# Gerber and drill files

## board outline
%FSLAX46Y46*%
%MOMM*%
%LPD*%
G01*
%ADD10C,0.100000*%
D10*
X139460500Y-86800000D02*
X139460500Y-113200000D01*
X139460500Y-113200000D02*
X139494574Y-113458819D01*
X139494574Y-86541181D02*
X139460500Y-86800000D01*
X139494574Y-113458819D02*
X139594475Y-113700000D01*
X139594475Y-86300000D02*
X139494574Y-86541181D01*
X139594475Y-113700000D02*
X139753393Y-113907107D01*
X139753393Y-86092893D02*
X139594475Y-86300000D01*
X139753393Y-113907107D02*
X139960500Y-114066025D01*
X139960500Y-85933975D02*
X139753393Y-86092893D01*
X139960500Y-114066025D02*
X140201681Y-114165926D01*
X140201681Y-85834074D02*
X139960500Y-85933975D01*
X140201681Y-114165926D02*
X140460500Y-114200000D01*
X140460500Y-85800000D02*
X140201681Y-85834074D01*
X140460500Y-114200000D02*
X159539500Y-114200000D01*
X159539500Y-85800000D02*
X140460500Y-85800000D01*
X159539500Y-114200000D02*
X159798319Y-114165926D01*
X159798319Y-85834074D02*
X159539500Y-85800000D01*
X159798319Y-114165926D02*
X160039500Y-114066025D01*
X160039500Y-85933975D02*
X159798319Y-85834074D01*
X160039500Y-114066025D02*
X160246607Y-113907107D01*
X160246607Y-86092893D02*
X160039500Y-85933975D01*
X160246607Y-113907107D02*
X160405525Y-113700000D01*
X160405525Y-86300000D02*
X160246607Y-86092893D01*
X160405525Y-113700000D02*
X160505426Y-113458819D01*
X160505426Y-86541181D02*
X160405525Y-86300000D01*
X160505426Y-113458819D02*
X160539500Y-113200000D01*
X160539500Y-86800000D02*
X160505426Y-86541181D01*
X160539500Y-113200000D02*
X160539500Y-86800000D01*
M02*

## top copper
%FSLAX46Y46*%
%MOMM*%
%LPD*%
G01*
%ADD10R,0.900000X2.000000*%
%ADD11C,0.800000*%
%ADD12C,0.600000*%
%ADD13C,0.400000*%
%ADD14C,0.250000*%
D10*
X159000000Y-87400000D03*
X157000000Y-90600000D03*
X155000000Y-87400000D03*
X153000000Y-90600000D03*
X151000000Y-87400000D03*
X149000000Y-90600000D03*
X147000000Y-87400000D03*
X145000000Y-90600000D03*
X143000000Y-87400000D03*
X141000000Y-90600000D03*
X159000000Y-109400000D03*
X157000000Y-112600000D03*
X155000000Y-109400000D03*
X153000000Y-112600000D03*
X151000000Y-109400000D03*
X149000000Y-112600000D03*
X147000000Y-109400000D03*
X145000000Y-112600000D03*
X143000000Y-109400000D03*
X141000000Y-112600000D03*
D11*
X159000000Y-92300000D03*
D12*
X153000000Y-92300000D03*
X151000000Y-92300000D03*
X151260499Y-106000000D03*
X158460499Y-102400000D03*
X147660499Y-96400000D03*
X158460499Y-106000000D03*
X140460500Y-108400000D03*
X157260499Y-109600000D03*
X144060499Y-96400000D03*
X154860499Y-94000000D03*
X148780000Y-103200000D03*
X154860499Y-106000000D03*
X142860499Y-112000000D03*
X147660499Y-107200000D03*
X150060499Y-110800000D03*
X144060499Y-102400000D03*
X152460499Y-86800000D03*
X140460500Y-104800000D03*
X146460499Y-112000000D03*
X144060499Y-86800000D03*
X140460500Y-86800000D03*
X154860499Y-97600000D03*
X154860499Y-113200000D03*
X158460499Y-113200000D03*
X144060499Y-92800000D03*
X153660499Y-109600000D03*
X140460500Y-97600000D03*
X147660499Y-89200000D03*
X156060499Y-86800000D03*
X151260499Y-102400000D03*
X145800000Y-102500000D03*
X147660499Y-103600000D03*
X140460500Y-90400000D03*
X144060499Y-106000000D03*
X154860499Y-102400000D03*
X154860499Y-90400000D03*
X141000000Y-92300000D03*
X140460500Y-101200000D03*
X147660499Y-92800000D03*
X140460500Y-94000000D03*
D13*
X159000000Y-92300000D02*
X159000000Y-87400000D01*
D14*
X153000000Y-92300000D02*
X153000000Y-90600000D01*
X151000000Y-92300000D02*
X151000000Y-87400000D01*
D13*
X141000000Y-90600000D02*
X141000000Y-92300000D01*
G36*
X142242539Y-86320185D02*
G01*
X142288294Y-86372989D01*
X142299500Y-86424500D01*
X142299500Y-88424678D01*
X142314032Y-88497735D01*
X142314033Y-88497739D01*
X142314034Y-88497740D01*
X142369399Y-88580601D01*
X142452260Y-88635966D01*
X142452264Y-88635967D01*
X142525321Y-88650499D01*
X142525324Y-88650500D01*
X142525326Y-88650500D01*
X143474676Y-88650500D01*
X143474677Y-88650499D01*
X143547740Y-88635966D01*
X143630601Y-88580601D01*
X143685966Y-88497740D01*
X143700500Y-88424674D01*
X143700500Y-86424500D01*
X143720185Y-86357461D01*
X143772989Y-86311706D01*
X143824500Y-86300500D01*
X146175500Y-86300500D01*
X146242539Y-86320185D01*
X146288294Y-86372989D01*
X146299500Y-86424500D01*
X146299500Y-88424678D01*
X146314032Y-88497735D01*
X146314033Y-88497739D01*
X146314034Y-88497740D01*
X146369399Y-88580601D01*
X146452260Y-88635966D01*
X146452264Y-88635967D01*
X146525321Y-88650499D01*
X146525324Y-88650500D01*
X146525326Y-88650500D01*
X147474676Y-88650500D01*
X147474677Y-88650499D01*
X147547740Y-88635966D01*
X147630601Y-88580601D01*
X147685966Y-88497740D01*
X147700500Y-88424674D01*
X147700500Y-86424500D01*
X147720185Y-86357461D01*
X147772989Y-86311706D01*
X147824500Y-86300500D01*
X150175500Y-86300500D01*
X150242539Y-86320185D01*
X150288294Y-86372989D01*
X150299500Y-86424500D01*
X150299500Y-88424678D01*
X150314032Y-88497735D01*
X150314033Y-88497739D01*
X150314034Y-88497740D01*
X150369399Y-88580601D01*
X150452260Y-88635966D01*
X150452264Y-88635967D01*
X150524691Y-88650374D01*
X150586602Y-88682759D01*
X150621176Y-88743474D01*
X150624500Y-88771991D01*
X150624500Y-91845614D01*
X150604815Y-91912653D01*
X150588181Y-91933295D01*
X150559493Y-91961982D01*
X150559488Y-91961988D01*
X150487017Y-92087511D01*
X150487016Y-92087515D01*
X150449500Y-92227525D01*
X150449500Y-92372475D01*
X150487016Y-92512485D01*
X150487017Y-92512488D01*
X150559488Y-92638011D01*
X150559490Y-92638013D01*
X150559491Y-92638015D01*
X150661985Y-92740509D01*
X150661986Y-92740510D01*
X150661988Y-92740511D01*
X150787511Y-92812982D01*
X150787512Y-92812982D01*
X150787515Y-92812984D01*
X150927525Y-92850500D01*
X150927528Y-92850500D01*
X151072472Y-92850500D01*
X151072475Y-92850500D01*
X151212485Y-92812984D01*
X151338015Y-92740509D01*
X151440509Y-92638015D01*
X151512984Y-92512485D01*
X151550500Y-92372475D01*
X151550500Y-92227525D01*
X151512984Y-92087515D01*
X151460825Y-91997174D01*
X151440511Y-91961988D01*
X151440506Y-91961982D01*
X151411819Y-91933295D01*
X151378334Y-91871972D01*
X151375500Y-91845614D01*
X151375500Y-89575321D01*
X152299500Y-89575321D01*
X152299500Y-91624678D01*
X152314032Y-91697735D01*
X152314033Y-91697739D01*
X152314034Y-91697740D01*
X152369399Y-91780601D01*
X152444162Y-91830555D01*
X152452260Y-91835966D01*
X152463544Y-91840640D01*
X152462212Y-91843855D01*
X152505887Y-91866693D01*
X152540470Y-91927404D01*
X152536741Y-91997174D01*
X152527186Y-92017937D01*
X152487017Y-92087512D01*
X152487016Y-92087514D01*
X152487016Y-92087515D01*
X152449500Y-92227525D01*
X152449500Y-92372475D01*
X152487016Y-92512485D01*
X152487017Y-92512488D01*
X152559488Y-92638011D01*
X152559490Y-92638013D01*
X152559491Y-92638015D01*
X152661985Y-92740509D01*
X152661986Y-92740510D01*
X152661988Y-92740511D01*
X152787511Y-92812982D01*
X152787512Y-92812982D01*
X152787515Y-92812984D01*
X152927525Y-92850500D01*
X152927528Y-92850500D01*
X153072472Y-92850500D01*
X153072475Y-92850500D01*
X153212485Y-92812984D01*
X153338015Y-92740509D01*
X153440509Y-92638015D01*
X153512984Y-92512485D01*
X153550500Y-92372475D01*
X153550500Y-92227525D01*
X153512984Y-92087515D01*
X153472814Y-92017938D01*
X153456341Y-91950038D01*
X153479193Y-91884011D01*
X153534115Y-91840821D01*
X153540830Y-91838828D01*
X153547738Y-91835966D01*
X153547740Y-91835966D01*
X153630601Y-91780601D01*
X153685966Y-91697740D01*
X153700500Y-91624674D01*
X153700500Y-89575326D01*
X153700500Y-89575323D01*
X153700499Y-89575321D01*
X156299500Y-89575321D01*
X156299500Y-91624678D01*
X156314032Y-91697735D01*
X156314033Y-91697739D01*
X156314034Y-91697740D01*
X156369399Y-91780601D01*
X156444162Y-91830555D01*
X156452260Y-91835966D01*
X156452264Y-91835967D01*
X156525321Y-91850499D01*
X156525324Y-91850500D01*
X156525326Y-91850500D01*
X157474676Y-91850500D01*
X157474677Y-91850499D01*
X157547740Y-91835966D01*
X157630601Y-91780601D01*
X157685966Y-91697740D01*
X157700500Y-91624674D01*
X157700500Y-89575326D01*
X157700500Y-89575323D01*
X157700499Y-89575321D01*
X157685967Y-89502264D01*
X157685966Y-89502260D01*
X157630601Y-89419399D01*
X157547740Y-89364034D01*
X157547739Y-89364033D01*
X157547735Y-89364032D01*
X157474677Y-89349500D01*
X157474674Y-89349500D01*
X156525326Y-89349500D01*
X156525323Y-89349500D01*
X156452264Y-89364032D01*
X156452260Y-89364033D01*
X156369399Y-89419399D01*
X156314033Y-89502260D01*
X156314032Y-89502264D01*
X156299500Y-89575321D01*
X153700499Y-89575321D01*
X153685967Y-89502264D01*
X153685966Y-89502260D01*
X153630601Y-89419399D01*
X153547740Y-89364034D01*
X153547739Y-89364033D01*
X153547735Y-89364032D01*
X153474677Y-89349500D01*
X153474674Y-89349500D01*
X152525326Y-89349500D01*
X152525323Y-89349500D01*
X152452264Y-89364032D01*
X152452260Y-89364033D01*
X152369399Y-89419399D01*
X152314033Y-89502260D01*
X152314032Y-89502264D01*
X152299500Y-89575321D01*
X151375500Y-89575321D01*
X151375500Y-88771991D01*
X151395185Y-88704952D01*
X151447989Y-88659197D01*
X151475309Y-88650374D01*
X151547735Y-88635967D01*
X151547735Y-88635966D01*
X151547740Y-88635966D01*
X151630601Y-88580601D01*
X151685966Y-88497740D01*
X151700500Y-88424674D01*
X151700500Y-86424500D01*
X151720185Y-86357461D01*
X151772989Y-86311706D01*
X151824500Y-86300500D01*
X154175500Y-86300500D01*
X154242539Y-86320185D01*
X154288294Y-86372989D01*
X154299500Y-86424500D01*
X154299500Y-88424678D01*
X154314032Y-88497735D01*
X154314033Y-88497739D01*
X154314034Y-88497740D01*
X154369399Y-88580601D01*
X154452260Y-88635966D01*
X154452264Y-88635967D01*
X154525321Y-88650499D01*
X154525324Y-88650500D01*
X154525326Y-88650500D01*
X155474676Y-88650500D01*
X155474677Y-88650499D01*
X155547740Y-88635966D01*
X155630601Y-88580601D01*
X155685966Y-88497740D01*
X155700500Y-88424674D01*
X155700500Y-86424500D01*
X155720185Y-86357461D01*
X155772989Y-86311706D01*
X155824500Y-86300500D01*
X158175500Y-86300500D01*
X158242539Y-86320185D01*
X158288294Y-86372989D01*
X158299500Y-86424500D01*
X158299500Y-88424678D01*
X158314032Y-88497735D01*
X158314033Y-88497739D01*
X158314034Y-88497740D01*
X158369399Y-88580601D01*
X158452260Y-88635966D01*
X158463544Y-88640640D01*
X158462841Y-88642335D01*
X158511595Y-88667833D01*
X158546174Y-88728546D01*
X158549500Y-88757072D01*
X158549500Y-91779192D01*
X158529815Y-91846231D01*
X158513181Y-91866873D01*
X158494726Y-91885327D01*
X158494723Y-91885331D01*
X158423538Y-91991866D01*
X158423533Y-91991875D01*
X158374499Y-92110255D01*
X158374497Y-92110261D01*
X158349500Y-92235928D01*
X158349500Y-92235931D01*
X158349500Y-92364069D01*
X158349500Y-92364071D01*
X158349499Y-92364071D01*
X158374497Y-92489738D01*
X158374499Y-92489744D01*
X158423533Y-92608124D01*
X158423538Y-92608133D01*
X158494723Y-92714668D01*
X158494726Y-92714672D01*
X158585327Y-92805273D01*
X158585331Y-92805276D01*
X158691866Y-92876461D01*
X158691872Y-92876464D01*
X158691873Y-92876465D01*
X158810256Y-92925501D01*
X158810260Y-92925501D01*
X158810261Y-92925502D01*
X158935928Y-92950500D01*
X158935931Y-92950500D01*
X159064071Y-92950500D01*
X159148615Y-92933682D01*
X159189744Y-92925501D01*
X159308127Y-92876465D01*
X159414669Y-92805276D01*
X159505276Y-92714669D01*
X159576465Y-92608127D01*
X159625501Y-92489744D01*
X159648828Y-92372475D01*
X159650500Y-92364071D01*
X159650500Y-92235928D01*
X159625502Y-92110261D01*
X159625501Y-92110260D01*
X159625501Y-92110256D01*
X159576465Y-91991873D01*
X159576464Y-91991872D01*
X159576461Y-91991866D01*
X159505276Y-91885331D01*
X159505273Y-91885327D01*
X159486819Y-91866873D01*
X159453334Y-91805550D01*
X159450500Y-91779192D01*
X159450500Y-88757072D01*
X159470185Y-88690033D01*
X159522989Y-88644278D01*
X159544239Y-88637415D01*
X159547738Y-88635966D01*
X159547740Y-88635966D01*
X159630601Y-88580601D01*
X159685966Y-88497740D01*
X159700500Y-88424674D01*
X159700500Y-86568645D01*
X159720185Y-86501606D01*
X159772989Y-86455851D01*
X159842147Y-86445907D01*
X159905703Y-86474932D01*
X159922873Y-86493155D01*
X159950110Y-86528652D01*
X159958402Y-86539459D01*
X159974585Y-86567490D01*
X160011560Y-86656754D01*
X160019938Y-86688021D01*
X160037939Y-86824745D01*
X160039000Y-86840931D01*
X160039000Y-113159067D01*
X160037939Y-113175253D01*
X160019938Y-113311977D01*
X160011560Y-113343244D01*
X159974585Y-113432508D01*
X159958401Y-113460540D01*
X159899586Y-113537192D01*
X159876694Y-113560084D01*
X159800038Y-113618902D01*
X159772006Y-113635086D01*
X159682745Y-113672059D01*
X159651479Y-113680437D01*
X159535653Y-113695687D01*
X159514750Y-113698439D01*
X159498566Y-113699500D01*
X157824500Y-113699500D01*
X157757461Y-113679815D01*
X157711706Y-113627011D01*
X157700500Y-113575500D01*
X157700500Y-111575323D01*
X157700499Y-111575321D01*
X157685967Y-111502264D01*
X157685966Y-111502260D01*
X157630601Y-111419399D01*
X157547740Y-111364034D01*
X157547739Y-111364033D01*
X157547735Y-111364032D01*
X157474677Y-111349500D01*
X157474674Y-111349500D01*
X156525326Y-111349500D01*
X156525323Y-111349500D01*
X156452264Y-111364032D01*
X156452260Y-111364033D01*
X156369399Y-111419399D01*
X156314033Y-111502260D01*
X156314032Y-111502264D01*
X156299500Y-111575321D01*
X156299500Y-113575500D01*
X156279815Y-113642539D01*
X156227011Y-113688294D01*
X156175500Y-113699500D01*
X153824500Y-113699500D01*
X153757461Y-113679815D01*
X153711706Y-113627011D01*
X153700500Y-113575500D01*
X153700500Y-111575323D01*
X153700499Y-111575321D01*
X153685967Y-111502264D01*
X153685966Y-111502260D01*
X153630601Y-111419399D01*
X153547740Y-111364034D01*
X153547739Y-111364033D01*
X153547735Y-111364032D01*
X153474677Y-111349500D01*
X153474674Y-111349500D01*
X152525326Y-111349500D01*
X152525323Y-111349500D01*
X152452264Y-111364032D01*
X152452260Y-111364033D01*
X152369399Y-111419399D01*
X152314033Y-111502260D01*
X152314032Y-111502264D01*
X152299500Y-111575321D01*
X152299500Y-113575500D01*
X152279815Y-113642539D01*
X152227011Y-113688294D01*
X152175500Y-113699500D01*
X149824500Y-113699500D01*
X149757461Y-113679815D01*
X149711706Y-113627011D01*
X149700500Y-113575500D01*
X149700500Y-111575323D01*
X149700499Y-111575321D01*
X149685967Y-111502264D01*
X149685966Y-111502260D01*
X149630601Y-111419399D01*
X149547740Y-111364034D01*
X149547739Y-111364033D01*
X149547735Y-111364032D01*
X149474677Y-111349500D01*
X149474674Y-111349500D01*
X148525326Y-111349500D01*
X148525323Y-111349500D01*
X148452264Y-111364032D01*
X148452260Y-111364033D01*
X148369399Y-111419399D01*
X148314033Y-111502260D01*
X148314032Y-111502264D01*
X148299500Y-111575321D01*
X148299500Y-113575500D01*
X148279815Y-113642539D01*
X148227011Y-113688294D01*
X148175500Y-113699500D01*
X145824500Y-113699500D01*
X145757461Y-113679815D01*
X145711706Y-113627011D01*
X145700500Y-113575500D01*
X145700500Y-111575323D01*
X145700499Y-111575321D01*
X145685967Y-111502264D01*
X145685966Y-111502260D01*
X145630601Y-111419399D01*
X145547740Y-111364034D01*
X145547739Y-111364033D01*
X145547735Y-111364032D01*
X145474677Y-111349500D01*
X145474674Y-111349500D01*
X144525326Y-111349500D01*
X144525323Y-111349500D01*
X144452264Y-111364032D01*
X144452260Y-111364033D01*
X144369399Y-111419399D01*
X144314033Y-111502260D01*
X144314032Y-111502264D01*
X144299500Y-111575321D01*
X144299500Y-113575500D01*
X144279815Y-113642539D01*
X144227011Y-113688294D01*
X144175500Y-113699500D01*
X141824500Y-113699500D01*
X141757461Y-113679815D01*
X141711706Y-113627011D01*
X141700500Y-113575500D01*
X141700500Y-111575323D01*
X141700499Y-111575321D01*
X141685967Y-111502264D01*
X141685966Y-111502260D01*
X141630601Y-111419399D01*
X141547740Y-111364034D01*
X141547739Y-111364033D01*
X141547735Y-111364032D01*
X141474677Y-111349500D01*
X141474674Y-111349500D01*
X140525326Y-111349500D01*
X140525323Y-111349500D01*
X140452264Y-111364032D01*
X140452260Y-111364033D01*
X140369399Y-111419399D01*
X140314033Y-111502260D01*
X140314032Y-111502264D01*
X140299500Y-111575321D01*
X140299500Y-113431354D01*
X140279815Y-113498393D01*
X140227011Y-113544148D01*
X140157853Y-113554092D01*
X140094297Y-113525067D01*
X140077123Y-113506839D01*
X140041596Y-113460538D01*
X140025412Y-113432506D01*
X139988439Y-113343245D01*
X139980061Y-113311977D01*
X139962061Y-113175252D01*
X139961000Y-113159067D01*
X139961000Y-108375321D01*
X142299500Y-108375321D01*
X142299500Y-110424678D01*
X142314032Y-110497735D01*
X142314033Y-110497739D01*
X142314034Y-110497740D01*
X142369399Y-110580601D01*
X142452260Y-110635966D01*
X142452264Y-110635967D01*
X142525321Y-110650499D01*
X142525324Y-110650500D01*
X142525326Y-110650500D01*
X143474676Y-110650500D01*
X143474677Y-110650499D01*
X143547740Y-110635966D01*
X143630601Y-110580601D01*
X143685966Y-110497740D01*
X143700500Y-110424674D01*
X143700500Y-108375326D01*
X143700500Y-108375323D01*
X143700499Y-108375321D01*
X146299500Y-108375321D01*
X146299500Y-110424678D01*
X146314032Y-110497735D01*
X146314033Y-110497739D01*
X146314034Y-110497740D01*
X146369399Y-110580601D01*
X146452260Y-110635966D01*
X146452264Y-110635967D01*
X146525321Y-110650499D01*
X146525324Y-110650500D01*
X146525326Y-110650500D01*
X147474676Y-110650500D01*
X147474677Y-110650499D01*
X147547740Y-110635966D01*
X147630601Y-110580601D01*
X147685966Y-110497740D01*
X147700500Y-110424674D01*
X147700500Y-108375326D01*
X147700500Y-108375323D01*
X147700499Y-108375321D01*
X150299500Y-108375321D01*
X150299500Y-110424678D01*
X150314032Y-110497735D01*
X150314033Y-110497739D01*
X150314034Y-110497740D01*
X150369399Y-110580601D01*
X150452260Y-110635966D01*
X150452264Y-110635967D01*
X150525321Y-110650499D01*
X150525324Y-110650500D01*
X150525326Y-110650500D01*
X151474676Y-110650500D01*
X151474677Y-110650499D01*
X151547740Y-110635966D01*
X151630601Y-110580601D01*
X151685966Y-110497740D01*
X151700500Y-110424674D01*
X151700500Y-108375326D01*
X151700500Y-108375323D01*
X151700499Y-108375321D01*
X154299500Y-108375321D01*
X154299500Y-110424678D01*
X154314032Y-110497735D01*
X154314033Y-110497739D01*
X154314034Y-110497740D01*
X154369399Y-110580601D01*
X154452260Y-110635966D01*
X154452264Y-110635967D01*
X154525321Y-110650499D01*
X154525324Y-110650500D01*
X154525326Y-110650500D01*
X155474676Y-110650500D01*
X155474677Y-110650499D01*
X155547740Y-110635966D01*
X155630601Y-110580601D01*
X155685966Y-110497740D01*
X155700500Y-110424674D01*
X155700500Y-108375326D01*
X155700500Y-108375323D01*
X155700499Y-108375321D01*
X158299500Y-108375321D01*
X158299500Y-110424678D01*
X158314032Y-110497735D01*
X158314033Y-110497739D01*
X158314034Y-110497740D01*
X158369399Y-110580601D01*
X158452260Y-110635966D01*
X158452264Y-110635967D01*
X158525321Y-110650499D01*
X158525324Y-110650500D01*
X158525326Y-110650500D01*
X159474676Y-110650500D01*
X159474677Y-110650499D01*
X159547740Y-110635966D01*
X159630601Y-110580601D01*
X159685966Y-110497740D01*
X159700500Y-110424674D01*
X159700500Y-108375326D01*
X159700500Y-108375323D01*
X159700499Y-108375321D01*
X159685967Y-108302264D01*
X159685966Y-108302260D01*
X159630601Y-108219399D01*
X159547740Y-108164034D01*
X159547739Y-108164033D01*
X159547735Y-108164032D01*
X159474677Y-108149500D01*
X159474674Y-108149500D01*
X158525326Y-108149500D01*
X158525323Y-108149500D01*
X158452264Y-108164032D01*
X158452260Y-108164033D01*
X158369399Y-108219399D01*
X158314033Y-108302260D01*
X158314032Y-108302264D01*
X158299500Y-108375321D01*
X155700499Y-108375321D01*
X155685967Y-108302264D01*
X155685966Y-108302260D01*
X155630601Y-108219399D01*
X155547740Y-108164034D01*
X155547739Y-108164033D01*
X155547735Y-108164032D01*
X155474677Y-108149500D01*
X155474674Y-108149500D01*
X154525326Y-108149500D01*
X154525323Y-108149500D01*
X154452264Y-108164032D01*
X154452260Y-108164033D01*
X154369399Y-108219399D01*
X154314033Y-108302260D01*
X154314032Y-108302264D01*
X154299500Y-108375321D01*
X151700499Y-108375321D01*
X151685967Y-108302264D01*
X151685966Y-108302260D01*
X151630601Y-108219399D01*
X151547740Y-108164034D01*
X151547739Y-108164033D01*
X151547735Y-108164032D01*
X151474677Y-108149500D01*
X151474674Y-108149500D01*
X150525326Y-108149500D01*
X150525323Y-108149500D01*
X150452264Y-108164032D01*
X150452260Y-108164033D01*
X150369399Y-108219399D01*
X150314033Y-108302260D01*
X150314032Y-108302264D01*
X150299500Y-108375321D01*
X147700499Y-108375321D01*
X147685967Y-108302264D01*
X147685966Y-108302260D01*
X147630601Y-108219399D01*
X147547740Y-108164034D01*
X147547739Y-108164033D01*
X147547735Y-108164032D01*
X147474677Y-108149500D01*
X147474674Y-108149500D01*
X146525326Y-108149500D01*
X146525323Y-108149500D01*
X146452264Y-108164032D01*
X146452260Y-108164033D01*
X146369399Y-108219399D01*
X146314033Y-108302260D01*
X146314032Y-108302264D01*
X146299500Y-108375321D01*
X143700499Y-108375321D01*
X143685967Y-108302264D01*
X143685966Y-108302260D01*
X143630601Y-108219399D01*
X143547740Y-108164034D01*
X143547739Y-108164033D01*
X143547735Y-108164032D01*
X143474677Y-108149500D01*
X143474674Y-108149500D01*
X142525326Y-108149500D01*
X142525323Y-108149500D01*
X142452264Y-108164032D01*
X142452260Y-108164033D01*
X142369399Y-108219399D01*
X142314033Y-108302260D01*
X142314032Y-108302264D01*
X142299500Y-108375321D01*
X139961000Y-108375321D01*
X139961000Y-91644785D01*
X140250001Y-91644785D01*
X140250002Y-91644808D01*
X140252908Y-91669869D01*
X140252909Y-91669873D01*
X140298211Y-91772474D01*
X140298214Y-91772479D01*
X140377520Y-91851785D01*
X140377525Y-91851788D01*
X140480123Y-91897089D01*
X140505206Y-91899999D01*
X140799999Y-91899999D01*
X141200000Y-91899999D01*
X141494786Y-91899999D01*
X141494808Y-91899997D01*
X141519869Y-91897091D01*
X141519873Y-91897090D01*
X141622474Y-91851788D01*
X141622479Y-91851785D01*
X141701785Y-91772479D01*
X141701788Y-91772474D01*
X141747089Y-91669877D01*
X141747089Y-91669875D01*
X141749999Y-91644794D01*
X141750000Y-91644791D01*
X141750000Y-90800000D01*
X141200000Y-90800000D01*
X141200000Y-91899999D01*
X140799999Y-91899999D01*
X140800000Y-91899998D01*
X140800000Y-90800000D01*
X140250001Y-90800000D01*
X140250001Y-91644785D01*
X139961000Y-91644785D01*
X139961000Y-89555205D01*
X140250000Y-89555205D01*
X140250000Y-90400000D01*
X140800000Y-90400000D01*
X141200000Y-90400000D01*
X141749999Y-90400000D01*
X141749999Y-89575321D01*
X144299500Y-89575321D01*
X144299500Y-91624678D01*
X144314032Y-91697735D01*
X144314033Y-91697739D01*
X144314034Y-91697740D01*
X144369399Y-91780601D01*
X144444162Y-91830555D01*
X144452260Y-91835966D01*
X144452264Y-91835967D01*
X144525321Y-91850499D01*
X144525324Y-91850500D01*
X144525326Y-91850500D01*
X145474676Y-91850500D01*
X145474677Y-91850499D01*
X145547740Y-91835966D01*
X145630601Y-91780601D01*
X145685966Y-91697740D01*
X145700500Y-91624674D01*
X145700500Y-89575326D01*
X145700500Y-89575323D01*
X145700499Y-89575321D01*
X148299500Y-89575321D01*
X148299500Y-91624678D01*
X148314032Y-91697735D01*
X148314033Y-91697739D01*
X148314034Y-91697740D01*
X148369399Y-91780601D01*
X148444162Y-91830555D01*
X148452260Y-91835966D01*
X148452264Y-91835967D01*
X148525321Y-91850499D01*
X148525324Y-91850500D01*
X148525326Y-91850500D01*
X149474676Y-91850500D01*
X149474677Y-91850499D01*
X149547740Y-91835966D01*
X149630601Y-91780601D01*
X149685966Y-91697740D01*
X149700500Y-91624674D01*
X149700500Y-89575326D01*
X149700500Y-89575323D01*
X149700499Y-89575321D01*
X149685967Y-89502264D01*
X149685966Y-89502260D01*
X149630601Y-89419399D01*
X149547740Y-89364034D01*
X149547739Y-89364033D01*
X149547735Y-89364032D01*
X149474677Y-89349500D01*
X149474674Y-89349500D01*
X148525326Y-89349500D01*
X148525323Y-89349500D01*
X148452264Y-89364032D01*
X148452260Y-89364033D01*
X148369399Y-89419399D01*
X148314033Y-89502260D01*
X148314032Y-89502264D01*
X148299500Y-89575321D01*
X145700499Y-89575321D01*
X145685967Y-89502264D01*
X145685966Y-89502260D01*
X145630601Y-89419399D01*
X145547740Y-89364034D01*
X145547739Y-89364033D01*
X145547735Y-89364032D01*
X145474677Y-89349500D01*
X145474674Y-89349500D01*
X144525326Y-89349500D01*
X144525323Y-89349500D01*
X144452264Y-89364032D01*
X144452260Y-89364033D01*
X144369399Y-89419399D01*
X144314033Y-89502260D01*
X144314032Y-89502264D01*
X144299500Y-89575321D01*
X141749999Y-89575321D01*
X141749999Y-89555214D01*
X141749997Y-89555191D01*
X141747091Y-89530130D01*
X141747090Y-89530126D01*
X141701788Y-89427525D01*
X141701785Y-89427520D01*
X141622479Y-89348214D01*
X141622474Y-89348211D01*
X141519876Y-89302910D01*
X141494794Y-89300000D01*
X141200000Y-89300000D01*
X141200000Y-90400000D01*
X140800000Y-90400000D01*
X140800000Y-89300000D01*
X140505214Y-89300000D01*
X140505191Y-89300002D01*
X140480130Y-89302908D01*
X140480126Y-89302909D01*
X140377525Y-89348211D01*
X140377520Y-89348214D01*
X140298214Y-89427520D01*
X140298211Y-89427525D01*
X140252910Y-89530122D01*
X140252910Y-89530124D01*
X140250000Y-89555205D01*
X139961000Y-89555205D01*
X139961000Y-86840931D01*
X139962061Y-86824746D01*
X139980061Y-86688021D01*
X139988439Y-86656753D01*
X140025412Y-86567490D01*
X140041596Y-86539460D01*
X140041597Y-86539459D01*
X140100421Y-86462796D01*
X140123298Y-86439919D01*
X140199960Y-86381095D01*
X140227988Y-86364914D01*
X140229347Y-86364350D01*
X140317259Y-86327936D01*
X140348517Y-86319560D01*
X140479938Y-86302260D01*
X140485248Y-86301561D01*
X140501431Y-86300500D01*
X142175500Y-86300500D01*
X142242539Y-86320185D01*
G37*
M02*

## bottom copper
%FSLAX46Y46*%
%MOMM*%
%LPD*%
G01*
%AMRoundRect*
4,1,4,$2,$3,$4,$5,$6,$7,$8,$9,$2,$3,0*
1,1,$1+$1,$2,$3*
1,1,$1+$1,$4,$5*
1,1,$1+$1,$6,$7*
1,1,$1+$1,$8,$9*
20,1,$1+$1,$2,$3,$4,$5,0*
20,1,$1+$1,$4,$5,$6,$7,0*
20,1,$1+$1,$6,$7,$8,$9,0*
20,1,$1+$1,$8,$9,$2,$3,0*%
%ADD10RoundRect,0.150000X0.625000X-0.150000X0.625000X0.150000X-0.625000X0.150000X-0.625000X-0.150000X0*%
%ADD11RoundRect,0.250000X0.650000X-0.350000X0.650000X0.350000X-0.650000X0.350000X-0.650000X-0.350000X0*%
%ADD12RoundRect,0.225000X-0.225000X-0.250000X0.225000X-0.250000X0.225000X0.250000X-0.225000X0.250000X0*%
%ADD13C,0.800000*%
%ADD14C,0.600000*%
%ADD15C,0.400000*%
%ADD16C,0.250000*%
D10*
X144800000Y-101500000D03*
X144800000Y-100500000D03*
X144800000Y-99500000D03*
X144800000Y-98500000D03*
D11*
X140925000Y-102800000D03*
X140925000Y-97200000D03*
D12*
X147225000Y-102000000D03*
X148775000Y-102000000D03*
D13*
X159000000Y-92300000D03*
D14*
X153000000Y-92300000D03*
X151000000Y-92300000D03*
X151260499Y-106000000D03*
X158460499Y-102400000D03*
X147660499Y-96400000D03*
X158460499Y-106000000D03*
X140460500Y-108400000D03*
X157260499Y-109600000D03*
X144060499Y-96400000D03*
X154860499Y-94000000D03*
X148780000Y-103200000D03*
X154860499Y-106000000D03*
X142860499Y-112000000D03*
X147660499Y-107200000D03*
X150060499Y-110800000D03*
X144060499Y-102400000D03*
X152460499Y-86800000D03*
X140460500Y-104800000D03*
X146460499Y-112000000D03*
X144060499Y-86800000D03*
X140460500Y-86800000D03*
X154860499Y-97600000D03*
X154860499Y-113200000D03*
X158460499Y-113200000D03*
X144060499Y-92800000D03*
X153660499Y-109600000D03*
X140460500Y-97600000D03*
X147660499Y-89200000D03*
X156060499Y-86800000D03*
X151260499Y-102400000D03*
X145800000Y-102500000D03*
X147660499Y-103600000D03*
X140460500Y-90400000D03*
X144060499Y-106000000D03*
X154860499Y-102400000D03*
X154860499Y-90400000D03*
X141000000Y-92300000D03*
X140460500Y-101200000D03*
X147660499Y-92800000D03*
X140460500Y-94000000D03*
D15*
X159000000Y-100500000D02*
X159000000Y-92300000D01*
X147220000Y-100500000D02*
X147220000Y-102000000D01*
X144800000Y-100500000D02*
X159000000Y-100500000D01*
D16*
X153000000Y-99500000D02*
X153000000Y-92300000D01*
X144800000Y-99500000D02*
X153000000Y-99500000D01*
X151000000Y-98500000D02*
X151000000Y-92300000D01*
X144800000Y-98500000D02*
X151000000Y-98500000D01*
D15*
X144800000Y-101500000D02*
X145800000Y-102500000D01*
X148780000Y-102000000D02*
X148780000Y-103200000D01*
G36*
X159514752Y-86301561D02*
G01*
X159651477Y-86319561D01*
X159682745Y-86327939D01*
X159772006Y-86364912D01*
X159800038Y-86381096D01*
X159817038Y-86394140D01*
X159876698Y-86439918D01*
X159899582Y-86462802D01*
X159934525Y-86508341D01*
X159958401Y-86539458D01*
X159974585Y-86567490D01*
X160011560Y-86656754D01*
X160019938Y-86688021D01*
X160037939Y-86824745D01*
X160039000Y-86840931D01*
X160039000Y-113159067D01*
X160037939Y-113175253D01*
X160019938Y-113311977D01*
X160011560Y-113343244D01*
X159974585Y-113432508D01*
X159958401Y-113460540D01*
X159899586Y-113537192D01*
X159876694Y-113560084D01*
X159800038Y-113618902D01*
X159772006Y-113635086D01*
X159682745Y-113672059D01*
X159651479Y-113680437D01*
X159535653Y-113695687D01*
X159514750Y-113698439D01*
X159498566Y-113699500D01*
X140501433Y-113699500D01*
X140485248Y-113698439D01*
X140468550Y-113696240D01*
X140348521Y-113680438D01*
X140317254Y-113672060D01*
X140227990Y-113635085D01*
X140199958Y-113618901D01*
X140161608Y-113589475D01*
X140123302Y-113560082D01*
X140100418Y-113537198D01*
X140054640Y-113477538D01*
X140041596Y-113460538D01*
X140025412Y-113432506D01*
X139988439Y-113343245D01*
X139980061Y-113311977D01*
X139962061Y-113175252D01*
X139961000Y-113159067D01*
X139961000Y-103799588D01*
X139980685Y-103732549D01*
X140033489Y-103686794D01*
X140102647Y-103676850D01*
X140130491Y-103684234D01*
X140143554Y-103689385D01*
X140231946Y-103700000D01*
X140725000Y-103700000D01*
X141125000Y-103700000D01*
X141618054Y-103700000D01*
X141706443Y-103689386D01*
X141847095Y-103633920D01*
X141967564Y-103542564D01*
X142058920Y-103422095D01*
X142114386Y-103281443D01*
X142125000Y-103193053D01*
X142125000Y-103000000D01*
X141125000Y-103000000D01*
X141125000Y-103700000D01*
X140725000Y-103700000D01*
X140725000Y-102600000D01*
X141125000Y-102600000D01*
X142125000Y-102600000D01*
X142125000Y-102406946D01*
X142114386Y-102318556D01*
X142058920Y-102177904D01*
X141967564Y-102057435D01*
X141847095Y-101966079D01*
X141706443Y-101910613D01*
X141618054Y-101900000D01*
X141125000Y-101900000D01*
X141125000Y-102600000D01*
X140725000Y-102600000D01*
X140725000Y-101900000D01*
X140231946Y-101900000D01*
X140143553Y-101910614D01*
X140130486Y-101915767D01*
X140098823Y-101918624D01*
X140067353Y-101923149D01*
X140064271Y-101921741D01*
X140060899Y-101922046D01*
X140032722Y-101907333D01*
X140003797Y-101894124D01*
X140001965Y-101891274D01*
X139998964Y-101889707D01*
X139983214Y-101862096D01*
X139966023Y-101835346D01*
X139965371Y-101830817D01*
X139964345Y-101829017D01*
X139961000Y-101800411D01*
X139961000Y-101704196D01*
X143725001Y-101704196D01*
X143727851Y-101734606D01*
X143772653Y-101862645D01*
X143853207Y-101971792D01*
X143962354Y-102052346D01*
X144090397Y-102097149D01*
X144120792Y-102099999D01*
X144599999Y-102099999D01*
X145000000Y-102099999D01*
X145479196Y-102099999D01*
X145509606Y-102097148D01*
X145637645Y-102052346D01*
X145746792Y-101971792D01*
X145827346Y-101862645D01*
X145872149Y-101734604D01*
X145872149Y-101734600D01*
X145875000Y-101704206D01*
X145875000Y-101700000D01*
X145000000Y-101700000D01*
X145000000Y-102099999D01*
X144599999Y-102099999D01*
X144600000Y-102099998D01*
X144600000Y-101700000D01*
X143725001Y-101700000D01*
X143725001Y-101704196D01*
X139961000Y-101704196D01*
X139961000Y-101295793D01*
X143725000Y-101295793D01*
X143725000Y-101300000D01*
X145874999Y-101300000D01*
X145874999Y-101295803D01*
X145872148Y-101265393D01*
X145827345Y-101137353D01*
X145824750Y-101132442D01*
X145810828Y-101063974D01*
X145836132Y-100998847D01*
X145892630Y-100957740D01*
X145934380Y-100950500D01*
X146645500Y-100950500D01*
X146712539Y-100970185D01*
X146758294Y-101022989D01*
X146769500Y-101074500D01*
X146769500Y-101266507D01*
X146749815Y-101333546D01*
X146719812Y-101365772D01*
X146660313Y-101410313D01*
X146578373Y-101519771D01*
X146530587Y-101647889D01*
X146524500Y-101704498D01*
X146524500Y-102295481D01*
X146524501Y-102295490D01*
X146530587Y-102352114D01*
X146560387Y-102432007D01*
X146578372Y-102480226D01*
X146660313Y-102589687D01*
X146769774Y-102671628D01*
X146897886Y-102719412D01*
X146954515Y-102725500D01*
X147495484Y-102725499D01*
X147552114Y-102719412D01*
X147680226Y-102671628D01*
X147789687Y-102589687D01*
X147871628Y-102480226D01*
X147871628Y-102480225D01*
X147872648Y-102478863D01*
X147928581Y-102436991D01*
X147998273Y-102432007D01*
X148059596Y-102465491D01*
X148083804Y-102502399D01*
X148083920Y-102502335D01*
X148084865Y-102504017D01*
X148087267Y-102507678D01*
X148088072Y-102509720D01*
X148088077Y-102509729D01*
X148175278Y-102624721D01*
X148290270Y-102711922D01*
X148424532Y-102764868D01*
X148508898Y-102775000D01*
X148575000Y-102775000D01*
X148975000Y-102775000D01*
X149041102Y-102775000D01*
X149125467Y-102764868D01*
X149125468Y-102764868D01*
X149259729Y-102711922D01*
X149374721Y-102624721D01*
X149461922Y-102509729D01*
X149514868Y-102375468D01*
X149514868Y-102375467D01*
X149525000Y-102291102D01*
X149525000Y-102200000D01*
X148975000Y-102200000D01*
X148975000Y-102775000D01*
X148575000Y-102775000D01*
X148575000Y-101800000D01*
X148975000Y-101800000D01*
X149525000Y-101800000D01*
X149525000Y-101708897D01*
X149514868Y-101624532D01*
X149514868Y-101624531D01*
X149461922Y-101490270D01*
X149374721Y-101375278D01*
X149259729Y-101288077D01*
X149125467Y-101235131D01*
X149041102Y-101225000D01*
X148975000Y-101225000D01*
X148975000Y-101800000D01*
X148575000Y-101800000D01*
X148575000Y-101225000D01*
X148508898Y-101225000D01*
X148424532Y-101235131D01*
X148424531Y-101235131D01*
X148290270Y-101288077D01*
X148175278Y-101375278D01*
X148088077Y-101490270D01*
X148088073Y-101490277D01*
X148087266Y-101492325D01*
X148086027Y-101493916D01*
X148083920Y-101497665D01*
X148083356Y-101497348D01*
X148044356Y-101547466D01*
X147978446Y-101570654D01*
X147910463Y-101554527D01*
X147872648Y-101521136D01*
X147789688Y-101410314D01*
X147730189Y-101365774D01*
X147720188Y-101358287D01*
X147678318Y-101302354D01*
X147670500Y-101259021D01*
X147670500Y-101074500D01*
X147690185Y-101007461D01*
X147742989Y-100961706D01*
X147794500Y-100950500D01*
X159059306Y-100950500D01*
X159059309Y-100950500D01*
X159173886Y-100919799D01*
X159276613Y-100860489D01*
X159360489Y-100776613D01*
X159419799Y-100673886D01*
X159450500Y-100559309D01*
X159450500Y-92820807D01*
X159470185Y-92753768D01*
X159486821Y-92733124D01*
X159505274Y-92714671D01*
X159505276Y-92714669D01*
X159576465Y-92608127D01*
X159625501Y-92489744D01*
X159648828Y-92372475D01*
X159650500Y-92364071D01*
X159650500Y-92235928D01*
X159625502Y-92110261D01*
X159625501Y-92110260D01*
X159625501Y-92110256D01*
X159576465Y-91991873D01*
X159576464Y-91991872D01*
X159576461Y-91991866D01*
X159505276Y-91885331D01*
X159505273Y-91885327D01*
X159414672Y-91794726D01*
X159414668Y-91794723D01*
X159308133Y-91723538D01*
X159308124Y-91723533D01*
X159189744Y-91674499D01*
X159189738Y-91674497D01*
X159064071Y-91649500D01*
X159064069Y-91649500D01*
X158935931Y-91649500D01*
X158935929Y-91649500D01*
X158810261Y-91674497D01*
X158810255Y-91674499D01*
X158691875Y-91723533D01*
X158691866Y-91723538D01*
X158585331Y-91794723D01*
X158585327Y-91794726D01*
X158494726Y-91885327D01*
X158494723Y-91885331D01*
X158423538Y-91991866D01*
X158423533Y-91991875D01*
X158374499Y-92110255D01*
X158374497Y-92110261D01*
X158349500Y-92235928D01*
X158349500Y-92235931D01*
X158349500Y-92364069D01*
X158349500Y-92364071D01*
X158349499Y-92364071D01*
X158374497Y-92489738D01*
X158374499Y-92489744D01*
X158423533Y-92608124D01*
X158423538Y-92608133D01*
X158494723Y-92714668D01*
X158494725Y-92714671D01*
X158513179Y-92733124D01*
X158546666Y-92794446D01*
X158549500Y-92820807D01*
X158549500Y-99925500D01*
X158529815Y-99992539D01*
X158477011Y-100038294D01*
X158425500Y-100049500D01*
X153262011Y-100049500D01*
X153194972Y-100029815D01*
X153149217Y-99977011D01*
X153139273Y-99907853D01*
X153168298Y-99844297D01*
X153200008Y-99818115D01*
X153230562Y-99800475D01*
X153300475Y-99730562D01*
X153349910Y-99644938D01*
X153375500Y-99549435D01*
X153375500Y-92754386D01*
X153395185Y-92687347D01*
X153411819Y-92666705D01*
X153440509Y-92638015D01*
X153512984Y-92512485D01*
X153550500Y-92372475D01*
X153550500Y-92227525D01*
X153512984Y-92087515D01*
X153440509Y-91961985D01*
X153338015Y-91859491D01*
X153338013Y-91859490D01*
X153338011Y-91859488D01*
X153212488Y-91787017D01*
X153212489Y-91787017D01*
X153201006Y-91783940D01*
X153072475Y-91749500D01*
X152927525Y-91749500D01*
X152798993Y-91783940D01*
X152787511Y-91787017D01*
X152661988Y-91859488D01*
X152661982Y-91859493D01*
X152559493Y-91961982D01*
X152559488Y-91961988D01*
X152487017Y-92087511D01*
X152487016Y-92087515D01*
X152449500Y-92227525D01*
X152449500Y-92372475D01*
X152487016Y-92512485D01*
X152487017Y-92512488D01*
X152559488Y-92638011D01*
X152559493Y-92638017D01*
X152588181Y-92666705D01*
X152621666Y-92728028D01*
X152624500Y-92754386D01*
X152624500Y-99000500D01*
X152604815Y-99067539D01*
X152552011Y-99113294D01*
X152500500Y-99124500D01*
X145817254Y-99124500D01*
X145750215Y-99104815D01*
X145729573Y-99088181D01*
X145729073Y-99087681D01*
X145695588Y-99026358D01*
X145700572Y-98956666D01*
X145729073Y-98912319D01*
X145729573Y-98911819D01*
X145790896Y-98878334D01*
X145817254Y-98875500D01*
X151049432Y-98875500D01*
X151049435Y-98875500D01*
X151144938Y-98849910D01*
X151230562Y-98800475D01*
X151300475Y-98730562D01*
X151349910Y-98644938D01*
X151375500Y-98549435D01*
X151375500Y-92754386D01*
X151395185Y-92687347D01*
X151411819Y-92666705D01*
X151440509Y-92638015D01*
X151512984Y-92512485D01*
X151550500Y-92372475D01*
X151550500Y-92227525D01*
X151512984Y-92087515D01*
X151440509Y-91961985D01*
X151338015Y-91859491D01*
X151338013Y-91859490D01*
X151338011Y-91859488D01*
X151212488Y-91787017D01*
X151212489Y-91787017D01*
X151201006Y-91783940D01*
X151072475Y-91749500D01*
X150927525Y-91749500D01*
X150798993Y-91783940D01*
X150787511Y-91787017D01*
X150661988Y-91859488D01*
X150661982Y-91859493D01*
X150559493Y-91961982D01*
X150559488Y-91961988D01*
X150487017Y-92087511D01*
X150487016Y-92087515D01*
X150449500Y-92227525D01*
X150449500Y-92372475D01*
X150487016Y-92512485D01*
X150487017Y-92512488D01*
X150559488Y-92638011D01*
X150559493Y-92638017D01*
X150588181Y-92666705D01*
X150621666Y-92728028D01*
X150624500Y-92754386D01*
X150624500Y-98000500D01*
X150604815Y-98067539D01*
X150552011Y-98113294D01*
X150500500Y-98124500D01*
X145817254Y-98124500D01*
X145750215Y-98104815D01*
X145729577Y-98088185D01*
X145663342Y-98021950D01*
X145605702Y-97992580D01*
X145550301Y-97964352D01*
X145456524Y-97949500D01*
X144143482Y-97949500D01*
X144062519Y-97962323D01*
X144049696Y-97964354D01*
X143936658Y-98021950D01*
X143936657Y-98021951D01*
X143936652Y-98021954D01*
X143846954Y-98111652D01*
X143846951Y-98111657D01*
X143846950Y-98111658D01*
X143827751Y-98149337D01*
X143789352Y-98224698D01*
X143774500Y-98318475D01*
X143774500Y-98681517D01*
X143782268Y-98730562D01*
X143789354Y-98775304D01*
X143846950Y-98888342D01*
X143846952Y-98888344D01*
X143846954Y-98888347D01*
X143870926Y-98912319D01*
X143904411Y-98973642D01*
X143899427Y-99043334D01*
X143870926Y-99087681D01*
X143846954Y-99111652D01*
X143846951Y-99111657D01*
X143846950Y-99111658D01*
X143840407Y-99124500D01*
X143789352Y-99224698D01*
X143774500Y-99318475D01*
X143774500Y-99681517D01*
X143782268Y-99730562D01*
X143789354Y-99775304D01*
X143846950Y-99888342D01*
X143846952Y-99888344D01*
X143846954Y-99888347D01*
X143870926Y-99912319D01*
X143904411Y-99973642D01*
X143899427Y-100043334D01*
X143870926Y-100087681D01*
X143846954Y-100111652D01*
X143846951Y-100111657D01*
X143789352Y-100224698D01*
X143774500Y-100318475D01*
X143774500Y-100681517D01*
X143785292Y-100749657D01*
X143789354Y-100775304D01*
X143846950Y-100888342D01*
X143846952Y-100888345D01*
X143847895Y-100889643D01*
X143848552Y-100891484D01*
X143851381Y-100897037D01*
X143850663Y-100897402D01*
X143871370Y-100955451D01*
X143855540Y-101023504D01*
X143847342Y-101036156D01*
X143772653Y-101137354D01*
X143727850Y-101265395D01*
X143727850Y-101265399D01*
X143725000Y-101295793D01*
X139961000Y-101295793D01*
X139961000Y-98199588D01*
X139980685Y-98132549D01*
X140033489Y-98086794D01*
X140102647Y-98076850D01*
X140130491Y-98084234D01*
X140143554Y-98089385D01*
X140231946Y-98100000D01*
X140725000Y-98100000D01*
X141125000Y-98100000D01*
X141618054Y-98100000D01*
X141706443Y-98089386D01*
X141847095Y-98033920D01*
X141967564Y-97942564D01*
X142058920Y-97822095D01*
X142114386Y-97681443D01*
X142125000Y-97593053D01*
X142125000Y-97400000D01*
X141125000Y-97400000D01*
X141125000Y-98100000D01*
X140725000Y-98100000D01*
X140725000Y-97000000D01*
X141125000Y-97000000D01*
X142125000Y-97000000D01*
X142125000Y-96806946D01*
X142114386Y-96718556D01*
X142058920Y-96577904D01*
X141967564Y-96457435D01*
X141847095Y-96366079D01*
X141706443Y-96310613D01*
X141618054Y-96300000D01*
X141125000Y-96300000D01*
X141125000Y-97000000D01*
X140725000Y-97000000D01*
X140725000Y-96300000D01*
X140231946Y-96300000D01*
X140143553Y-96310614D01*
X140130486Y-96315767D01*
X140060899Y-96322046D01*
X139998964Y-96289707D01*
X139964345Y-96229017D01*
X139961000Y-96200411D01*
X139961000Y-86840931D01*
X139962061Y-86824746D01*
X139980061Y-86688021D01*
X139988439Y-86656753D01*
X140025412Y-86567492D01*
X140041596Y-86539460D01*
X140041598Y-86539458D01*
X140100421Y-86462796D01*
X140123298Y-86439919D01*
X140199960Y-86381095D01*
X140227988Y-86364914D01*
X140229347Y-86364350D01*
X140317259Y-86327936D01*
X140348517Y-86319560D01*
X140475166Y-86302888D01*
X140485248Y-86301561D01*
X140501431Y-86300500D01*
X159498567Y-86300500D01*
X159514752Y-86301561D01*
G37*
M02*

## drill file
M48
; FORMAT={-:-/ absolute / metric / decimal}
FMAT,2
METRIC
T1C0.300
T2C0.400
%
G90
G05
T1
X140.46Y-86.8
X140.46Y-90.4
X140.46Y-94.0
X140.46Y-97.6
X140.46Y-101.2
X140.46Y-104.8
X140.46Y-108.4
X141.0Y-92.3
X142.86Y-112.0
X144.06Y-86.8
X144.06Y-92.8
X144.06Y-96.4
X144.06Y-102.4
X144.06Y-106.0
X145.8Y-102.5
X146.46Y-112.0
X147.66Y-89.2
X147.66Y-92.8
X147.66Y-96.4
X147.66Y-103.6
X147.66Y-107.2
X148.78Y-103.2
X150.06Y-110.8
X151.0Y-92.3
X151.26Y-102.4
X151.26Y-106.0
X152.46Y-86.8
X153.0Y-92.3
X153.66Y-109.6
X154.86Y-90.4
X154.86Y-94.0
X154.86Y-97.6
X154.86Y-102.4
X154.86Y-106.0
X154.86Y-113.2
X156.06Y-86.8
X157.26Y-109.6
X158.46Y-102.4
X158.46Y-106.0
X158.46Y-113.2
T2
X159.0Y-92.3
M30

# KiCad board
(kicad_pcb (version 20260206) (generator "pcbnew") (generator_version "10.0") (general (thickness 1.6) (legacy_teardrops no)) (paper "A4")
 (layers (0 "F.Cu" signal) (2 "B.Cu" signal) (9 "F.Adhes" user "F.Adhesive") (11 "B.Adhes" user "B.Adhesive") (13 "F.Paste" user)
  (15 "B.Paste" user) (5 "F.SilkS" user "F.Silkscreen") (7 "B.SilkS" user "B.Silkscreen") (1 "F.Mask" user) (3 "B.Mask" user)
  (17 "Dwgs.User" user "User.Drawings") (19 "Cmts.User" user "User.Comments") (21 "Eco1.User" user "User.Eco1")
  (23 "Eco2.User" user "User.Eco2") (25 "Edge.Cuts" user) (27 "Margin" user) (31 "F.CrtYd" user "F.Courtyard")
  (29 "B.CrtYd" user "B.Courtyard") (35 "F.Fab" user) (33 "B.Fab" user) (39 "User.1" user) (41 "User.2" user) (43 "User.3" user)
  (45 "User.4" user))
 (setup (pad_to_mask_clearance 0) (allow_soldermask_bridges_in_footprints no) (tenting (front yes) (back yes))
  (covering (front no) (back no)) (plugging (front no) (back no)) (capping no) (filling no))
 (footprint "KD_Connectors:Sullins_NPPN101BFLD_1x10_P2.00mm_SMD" (layer "F.Cu") (at 150 89 180)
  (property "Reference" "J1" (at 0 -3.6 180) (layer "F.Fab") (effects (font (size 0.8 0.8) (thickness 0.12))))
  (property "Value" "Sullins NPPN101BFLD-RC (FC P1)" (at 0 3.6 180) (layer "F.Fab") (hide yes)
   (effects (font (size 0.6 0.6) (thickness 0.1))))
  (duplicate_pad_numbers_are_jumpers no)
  (pad "1" smd rect (at -9 1.6 180) (size 0.9 2) (layers "F.Cu" "F.Mask" "F.Paste") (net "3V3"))
  (pad "2" smd rect (at -7 -1.6 180) (size 0.9 2) (layers "F.Cu" "F.Mask" "F.Paste"))
  (pad "3" smd rect (at -5 1.6 180) (size 0.9 2) (layers "F.Cu" "F.Mask" "F.Paste"))
  (pad "4" smd rect (at -3 -1.6 180) (size 0.9 2) (layers "F.Cu" "F.Mask" "F.Paste") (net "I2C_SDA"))
  (pad "5" smd rect (at -1 1.6 180) (size 0.9 2) (layers "F.Cu" "F.Mask" "F.Paste") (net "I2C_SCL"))
  (pad "6" smd rect (at 1 -1.6 180) (size 0.9 2) (layers "F.Cu" "F.Mask" "F.Paste"))
  (pad "7" smd rect (at 3 1.6 180) (size 0.9 2) (layers "F.Cu" "F.Mask" "F.Paste"))
  (pad "8" smd rect (at 5 -1.6 180) (size 0.9 2) (layers "F.Cu" "F.Mask" "F.Paste"))
  (pad "9" smd rect (at 7 1.6 180) (size 0.9 2) (layers "F.Cu" "F.Mask" "F.Paste"))
  (pad "10" smd rect (at 9 -1.6 180) (size 0.9 2) (layers "F.Cu" "F.Mask" "F.Paste") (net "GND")))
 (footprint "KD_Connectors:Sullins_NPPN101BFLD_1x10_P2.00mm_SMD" (layer "F.Cu") (at 150 111 180)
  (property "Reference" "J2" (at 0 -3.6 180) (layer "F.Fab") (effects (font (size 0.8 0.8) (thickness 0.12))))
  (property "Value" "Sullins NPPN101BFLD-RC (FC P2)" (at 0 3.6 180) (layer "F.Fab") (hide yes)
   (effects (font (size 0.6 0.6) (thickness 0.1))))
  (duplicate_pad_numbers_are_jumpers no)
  (pad "1" smd rect (at -9 1.6 180) (size 0.9 2) (layers "F.Cu" "F.Mask" "F.Paste"))
  (pad "2" smd rect (at -7 -1.6 180) (size 0.9 2) (layers "F.Cu" "F.Mask" "F.Paste"))
  (pad "3" smd rect (at -5 1.6 180) (size 0.9 2) (layers "F.Cu" "F.Mask" "F.Paste"))
  (pad "4" smd rect (at -3 -1.6 180) (size 0.9 2) (layers "F.Cu" "F.Mask" "F.Paste"))
  (pad "5" smd rect (at -1 1.6 180) (size 0.9 2) (layers "F.Cu" "F.Mask" "F.Paste"))
  (pad "6" smd rect (at 1 -1.6 180) (size 0.9 2) (layers "F.Cu" "F.Mask" "F.Paste"))
  (pad "7" smd rect (at 3 1.6 180) (size 0.9 2) (layers "F.Cu" "F.Mask" "F.Paste"))
  (pad "8" smd rect (at 5 -1.6 180) (size 0.9 2) (layers "F.Cu" "F.Mask" "F.Paste"))
  (pad "9" smd rect (at 7 1.6 180) (size 0.9 2) (layers "F.Cu" "F.Mask" "F.Paste"))
  (pad "10" smd rect (at 9 -1.6 180) (size 0.9 2) (layers "F.Cu" "F.Mask" "F.Paste")))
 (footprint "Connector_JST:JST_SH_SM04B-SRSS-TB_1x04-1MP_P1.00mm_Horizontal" (layer "B.Cu") (at 142.8 100 90)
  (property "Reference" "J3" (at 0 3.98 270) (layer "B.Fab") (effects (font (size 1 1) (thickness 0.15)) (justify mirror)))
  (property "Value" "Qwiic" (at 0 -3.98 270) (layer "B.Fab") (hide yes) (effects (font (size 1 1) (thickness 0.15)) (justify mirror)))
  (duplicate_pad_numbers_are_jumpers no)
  (pad "1" smd roundrect (at -1.5 2 90) (size 0.6 1.55) (layers "B.Cu" "B.Mask" "B.Paste") (roundrect_rratio 0.25) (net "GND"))
  (pad "2" smd roundrect (at -0.5 2 90) (size 0.6 1.55) (layers "B.Cu" "B.Mask" "B.Paste") (roundrect_rratio 0.25) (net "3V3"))
  (pad "3" smd roundrect (at 0.5 2 90) (size 0.6 1.55) (layers "B.Cu" "B.Mask" "B.Paste") (roundrect_rratio 0.25) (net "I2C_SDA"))
  (pad "4" smd roundrect (at 1.5 2 90) (size 0.6 1.55) (layers "B.Cu" "B.Mask" "B.Paste") (roundrect_rratio 0.25) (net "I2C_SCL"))
  (pad "MP" smd roundrect (at -2.8 -1.875 90) (size 1.2 1.8) (layers "B.Cu" "B.Mask" "B.Paste") (roundrect_rratio 0.208333) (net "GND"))
  (pad "MP" smd roundrect (at 2.8 -1.875 90) (size 1.2 1.8) (layers "B.Cu" "B.Mask" "B.Paste") (roundrect_rratio 0.208333) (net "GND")))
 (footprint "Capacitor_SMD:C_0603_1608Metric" (layer "B.Cu") (at 148 102)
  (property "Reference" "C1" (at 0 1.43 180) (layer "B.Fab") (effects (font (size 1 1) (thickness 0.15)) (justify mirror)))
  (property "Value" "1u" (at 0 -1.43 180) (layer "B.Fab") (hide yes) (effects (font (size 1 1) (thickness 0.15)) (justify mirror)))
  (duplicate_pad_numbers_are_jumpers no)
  (pad "1" smd roundrect (at -0.775 0) (size 0.9 0.95) (layers "B.Cu" "B.Mask" "B.Paste") (roundrect_rratio 0.25) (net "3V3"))
  (pad "2" smd roundrect (at 0.775 0) (size 0.9 0.95) (layers "B.Cu" "B.Mask" "B.Paste") (roundrect_rratio 0.25) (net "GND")))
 (gr_line (start 139.4605 86.8) (end 139.4605 113.2) (stroke (width 0.1) (type default)) (layer "Edge.Cuts"))
 (gr_line (start 139.4605 113.2) (end 139.494574 113.458819) (stroke (width 0.1) (type default)) (layer "Edge.Cuts"))
 (gr_line (start 139.494574 86.541181) (end 139.4605 86.8) (stroke (width 0.1) (type default)) (layer "Edge.Cuts"))
 (gr_line (start 139.494574 113.458819) (end 139.594475 113.7) (stroke (width 0.1) (type default)) (layer "Edge.Cuts"))
 (gr_line (start 139.594475 86.3) (end 139.494574 86.541181) (stroke (width 0.1) (type default)) (layer "Edge.Cuts"))
 (gr_line (start 139.594475 113.7) (end 139.753393 113.907107) (stroke (width 0.1) (type default)) (layer "Edge.Cuts"))
 (gr_line (start 139.753393 86.092893) (end 139.594475 86.3) (stroke (width 0.1) (type default)) (layer "Edge.Cuts"))
 (gr_line (start 139.753393 113.907107) (end 139.9605 114.066025) (stroke (width 0.1) (type default)) (layer "Edge.Cuts"))
 (gr_line (start 139.9605 85.933975) (end 139.753393 86.092893) (stroke (width 0.1) (type default)) (layer "Edge.Cuts"))
 (gr_line (start 139.9605 114.066025) (end 140.201681 114.165926) (stroke (width 0.1) (type default)) (layer "Edge.Cuts"))
 (gr_line (start 140.201681 85.834074) (end 139.9605 85.933975) (stroke (width 0.1) (type default)) (layer "Edge.Cuts"))
 (gr_line (start 140.201681 114.165926) (end 140.4605 114.2) (stroke (width 0.1) (type default)) (layer "Edge.Cuts"))
 (gr_line (start 140.4605 85.8) (end 140.201681 85.834074) (stroke (width 0.1) (type default)) (layer "Edge.Cuts"))
 (gr_line (start 140.4605 114.2) (end 159.5395 114.2) (stroke (width 0.1) (type default)) (layer "Edge.Cuts"))
 (gr_line (start 159.5395 85.8) (end 140.4605 85.8) (stroke (width 0.1) (type default)) (layer "Edge.Cuts"))
 (gr_line (start 159.5395 114.2) (end 159.798319 114.165926) (stroke (width 0.1) (type default)) (layer "Edge.Cuts"))
 (gr_line (start 159.798319 85.834074) (end 159.5395 85.8) (stroke (width 0.1) (type default)) (layer "Edge.Cuts"))
 (gr_line (start 159.798319 114.165926) (end 160.0395 114.066025) (stroke (width 0.1) (type default)) (layer "Edge.Cuts"))
 (gr_line (start 160.0395 85.933975) (end 159.798319 85.834074) (stroke (width 0.1) (type default)) (layer "Edge.Cuts"))
 (gr_line (start 160.0395 114.066025) (end 160.246607 113.907107) (stroke (width 0.1) (type default)) (layer "Edge.Cuts"))
 (gr_line (start 160.246607 86.092893) (end 160.0395 85.933975) (stroke (width 0.1) (type default)) (layer "Edge.Cuts"))
 (gr_line (start 160.246607 113.907107) (end 160.405525 113.7) (stroke (width 0.1) (type default)) (layer "Edge.Cuts"))
 (gr_line (start 160.405525 86.3) (end 160.246607 86.092893) (stroke (width 0.1) (type default)) (layer "Edge.Cuts"))
 (gr_line (start 160.405525 113.7) (end 160.505426 113.458819) (stroke (width 0.1) (type default)) (layer "Edge.Cuts"))
 (gr_line (start 160.505426 86.541181) (end 160.405525 86.3) (stroke (width 0.1) (type default)) (layer "Edge.Cuts"))
 (gr_line (start 160.505426 113.458819) (end 160.5395 113.2) (stroke (width 0.1) (type default)) (layer "Edge.Cuts"))
 (gr_line (start 160.5395 86.8) (end 160.505426 86.541181) (stroke (width 0.1) (type default)) (layer "Edge.Cuts"))
 (gr_line (start 160.5395 113.2) (end 160.5395 86.8) (stroke (width 0.1) (type default)) (layer "Edge.Cuts"))
 (segment (start 159 92.3) (end 159 87.4) (width 0.4) (layer "F.Cu") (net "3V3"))
 (via (at 159 92.3) (size 0.8) (drill 0.4) (layers "F.Cu" "B.Cu") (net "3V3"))
 (segment (start 159 100.5) (end 159 92.3) (width 0.4) (layer "B.Cu") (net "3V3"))
 (segment (start 147.22 100.5) (end 147.22 102) (width 0.4) (layer "B.Cu") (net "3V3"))
 (segment (start 144.8 100.5) (end 159 100.5) (width 0.4) (layer "B.Cu") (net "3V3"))
 (segment (start 153 92.3) (end 153 90.6) (width 0.25) (layer "F.Cu") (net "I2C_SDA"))
 (via (at 153 92.3) (size 0.6) (drill 0.3) (layers "F.Cu" "B.Cu") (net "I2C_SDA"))
 (segment (start 153 99.5) (end 153 92.3) (width 0.25) (layer "B.Cu") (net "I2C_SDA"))
 (segment (start 144.8 99.5) (end 153 99.5) (width 0.25) (layer "B.Cu") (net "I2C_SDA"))
 (segment (start 151 92.3) (end 151 87.4) (width 0.25) (layer "F.Cu") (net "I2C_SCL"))
 (via (at 151 92.3) (size 0.6) (drill 0.3) (layers "F.Cu" "B.Cu") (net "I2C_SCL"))
 (segment (start 151 98.5) (end 151 92.3) (width 0.25) (layer "B.Cu") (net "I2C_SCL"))
 (segment (start 144.8 98.5) (end 151 98.5) (width 0.25) (layer "B.Cu") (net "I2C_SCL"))
 (segment (start 141 90.6) (end 141 92.3) (width 0.4) (layer "F.Cu") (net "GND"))
 (via (at 151.260499 106) (size 0.6) (drill 0.3) (layers "F.Cu" "B.Cu") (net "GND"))
 (via (at 158.460499 102.4) (size 0.6) (drill 0.3) (layers "F.Cu" "B.Cu") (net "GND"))
 (via (at 147.660499 96.4) (size 0.6) (drill 0.3) (layers "F.Cu" "B.Cu") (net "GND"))
 (via (at 158.460499 106) (size 0.6) (drill 0.3) (layers "F.Cu" "B.Cu") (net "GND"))
 (via (at 140.4605 108.4) (size 0.6) (drill 0.3) (layers "F.Cu" "B.Cu") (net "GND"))
 (via (at 157.260499 109.6) (size 0.6) (drill 0.3) (layers "F.Cu" "B.Cu") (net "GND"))
 (via (at 144.060499 96.4) (size 0.6) (drill 0.3) (layers "F.Cu" "B.Cu") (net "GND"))
 (via (at 154.860499 94) (size 0.6) (drill 0.3) (layers "F.Cu" "B.Cu") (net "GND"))
 (via (at 148.78 103.2) (size 0.6) (drill 0.3) (layers "F.Cu" "B.Cu") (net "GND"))
 (via (at 154.860499 106) (size 0.6) (drill 0.3) (layers "F.Cu" "B.Cu") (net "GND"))
 (via (at 142.860499 112) (size 0.6) (drill 0.3) (layers "F.Cu" "B.Cu") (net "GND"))
 (via (at 147.660499 107.2) (size 0.6) (drill 0.3) (layers "F.Cu" "B.Cu") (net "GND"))
 (via (at 150.060499 110.8) (size 0.6) (drill 0.3) (layers "F.Cu" "B.Cu") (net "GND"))
 (via (at 144.060499 102.4) (size 0.6) (drill 0.3) (layers "F.Cu" "B.Cu") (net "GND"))
 (via (at 152.460499 86.8) (size 0.6) (drill 0.3) (layers "F.Cu" "B.Cu") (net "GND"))
 (via (at 140.4605 104.8) (size 0.6) (drill 0.3) (layers "F.Cu" "B.Cu") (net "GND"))
 (via (at 146.460499 112) (size 0.6) (drill 0.3) (layers "F.Cu" "B.Cu") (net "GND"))
 (via (at 144.060499 86.8) (size 0.6) (drill 0.3) (layers "F.Cu" "B.Cu") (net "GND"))
 (via (at 140.4605 86.8) (size 0.6) (drill 0.3) (layers "F.Cu" "B.Cu") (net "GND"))
 (via (at 154.860499 97.6) (size 0.6) (drill 0.3) (layers "F.Cu" "B.Cu") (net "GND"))
 (via (at 154.860499 113.2) (size 0.6) (drill 0.3) (layers "F.Cu" "B.Cu") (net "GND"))
 (via (at 158.460499 113.2) (size 0.6) (drill 0.3) (layers "F.Cu" "B.Cu") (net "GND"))
 (via (at 144.060499 92.8) (size 0.6) (drill 0.3) (layers "F.Cu" "B.Cu") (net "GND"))
 (via (at 153.660499 109.6) (size 0.6) (drill 0.3) (layers "F.Cu" "B.Cu") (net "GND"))
 (via (at 140.4605 97.6) (size 0.6) (drill 0.3) (layers "F.Cu" "B.Cu") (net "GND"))
 (via (at 147.660499 89.2) (size 0.6) (drill 0.3) (layers "F.Cu" "B.Cu") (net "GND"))
 (via (at 156.060499 86.8) (size 0.6) (drill 0.3) (layers "F.Cu" "B.Cu") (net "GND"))
 (via (at 151.260499 102.4) (size 0.6) (drill 0.3) (layers "F.Cu" "B.Cu") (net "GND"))
 (via (at 145.8 102.5) (size 0.6) (drill 0.3) (layers "F.Cu" "B.Cu") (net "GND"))
 (via (at 147.660499 103.6) (size 0.6) (drill 0.3) (layers "F.Cu" "B.Cu") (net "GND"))
 (via (at 140.4605 90.4) (size 0.6) (drill 0.3) (layers "F.Cu" "B.Cu") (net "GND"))
 (via (at 144.060499 106) (size 0.6) (drill 0.3) (layers "F.Cu" "B.Cu") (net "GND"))
 (via (at 154.860499 102.4) (size 0.6) (drill 0.3) (layers "F.Cu" "B.Cu") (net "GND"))
 (via (at 154.860499 90.4) (size 0.6) (drill 0.3) (layers "F.Cu" "B.Cu") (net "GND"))
 (via (at 141 92.3) (size 0.6) (drill 0.3) (layers "F.Cu" "B.Cu") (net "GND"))
 (via (at 140.4605 101.2) (size 0.6) (drill 0.3) (layers "F.Cu" "B.Cu") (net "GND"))
 (via (at 147.660499 92.8) (size 0.6) (drill 0.3) (layers "F.Cu" "B.Cu") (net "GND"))
 (via (at 140.4605 94) (size 0.6) (drill 0.3) (layers "F.Cu" "B.Cu") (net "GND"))
 (segment (start 144.8 101.5) (end 145.8 102.5) (width 0.4) (layer "B.Cu") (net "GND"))
 (segment (start 148.78 102) (end 148.78 103.2) (width 0.4) (layer "B.Cu") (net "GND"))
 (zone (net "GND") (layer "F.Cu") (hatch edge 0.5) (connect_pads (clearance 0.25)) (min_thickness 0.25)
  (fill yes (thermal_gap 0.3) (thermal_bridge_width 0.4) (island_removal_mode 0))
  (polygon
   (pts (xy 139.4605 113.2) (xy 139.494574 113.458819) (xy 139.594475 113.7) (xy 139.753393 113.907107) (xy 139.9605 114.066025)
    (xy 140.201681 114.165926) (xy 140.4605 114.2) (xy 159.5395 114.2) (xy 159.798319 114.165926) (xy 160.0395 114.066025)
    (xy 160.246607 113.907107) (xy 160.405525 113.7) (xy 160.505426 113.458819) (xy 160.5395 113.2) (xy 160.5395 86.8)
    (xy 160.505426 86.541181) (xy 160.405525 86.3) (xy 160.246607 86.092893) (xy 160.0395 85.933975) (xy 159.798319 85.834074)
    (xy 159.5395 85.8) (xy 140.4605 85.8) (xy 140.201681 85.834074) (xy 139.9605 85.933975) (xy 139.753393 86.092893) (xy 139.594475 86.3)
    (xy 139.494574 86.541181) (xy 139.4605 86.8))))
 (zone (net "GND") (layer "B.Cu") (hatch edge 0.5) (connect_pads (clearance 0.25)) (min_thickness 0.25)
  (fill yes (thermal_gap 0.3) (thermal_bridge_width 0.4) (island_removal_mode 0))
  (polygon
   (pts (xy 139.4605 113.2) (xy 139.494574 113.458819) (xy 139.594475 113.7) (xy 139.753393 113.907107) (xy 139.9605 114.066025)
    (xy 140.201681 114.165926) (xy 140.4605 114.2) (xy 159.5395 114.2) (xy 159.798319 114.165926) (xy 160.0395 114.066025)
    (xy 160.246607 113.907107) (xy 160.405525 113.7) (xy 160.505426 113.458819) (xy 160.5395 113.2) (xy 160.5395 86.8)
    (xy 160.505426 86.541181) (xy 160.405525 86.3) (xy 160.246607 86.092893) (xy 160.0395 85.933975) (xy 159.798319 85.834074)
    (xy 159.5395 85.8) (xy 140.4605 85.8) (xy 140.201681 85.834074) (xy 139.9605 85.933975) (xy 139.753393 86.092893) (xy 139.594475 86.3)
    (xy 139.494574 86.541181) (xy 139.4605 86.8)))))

